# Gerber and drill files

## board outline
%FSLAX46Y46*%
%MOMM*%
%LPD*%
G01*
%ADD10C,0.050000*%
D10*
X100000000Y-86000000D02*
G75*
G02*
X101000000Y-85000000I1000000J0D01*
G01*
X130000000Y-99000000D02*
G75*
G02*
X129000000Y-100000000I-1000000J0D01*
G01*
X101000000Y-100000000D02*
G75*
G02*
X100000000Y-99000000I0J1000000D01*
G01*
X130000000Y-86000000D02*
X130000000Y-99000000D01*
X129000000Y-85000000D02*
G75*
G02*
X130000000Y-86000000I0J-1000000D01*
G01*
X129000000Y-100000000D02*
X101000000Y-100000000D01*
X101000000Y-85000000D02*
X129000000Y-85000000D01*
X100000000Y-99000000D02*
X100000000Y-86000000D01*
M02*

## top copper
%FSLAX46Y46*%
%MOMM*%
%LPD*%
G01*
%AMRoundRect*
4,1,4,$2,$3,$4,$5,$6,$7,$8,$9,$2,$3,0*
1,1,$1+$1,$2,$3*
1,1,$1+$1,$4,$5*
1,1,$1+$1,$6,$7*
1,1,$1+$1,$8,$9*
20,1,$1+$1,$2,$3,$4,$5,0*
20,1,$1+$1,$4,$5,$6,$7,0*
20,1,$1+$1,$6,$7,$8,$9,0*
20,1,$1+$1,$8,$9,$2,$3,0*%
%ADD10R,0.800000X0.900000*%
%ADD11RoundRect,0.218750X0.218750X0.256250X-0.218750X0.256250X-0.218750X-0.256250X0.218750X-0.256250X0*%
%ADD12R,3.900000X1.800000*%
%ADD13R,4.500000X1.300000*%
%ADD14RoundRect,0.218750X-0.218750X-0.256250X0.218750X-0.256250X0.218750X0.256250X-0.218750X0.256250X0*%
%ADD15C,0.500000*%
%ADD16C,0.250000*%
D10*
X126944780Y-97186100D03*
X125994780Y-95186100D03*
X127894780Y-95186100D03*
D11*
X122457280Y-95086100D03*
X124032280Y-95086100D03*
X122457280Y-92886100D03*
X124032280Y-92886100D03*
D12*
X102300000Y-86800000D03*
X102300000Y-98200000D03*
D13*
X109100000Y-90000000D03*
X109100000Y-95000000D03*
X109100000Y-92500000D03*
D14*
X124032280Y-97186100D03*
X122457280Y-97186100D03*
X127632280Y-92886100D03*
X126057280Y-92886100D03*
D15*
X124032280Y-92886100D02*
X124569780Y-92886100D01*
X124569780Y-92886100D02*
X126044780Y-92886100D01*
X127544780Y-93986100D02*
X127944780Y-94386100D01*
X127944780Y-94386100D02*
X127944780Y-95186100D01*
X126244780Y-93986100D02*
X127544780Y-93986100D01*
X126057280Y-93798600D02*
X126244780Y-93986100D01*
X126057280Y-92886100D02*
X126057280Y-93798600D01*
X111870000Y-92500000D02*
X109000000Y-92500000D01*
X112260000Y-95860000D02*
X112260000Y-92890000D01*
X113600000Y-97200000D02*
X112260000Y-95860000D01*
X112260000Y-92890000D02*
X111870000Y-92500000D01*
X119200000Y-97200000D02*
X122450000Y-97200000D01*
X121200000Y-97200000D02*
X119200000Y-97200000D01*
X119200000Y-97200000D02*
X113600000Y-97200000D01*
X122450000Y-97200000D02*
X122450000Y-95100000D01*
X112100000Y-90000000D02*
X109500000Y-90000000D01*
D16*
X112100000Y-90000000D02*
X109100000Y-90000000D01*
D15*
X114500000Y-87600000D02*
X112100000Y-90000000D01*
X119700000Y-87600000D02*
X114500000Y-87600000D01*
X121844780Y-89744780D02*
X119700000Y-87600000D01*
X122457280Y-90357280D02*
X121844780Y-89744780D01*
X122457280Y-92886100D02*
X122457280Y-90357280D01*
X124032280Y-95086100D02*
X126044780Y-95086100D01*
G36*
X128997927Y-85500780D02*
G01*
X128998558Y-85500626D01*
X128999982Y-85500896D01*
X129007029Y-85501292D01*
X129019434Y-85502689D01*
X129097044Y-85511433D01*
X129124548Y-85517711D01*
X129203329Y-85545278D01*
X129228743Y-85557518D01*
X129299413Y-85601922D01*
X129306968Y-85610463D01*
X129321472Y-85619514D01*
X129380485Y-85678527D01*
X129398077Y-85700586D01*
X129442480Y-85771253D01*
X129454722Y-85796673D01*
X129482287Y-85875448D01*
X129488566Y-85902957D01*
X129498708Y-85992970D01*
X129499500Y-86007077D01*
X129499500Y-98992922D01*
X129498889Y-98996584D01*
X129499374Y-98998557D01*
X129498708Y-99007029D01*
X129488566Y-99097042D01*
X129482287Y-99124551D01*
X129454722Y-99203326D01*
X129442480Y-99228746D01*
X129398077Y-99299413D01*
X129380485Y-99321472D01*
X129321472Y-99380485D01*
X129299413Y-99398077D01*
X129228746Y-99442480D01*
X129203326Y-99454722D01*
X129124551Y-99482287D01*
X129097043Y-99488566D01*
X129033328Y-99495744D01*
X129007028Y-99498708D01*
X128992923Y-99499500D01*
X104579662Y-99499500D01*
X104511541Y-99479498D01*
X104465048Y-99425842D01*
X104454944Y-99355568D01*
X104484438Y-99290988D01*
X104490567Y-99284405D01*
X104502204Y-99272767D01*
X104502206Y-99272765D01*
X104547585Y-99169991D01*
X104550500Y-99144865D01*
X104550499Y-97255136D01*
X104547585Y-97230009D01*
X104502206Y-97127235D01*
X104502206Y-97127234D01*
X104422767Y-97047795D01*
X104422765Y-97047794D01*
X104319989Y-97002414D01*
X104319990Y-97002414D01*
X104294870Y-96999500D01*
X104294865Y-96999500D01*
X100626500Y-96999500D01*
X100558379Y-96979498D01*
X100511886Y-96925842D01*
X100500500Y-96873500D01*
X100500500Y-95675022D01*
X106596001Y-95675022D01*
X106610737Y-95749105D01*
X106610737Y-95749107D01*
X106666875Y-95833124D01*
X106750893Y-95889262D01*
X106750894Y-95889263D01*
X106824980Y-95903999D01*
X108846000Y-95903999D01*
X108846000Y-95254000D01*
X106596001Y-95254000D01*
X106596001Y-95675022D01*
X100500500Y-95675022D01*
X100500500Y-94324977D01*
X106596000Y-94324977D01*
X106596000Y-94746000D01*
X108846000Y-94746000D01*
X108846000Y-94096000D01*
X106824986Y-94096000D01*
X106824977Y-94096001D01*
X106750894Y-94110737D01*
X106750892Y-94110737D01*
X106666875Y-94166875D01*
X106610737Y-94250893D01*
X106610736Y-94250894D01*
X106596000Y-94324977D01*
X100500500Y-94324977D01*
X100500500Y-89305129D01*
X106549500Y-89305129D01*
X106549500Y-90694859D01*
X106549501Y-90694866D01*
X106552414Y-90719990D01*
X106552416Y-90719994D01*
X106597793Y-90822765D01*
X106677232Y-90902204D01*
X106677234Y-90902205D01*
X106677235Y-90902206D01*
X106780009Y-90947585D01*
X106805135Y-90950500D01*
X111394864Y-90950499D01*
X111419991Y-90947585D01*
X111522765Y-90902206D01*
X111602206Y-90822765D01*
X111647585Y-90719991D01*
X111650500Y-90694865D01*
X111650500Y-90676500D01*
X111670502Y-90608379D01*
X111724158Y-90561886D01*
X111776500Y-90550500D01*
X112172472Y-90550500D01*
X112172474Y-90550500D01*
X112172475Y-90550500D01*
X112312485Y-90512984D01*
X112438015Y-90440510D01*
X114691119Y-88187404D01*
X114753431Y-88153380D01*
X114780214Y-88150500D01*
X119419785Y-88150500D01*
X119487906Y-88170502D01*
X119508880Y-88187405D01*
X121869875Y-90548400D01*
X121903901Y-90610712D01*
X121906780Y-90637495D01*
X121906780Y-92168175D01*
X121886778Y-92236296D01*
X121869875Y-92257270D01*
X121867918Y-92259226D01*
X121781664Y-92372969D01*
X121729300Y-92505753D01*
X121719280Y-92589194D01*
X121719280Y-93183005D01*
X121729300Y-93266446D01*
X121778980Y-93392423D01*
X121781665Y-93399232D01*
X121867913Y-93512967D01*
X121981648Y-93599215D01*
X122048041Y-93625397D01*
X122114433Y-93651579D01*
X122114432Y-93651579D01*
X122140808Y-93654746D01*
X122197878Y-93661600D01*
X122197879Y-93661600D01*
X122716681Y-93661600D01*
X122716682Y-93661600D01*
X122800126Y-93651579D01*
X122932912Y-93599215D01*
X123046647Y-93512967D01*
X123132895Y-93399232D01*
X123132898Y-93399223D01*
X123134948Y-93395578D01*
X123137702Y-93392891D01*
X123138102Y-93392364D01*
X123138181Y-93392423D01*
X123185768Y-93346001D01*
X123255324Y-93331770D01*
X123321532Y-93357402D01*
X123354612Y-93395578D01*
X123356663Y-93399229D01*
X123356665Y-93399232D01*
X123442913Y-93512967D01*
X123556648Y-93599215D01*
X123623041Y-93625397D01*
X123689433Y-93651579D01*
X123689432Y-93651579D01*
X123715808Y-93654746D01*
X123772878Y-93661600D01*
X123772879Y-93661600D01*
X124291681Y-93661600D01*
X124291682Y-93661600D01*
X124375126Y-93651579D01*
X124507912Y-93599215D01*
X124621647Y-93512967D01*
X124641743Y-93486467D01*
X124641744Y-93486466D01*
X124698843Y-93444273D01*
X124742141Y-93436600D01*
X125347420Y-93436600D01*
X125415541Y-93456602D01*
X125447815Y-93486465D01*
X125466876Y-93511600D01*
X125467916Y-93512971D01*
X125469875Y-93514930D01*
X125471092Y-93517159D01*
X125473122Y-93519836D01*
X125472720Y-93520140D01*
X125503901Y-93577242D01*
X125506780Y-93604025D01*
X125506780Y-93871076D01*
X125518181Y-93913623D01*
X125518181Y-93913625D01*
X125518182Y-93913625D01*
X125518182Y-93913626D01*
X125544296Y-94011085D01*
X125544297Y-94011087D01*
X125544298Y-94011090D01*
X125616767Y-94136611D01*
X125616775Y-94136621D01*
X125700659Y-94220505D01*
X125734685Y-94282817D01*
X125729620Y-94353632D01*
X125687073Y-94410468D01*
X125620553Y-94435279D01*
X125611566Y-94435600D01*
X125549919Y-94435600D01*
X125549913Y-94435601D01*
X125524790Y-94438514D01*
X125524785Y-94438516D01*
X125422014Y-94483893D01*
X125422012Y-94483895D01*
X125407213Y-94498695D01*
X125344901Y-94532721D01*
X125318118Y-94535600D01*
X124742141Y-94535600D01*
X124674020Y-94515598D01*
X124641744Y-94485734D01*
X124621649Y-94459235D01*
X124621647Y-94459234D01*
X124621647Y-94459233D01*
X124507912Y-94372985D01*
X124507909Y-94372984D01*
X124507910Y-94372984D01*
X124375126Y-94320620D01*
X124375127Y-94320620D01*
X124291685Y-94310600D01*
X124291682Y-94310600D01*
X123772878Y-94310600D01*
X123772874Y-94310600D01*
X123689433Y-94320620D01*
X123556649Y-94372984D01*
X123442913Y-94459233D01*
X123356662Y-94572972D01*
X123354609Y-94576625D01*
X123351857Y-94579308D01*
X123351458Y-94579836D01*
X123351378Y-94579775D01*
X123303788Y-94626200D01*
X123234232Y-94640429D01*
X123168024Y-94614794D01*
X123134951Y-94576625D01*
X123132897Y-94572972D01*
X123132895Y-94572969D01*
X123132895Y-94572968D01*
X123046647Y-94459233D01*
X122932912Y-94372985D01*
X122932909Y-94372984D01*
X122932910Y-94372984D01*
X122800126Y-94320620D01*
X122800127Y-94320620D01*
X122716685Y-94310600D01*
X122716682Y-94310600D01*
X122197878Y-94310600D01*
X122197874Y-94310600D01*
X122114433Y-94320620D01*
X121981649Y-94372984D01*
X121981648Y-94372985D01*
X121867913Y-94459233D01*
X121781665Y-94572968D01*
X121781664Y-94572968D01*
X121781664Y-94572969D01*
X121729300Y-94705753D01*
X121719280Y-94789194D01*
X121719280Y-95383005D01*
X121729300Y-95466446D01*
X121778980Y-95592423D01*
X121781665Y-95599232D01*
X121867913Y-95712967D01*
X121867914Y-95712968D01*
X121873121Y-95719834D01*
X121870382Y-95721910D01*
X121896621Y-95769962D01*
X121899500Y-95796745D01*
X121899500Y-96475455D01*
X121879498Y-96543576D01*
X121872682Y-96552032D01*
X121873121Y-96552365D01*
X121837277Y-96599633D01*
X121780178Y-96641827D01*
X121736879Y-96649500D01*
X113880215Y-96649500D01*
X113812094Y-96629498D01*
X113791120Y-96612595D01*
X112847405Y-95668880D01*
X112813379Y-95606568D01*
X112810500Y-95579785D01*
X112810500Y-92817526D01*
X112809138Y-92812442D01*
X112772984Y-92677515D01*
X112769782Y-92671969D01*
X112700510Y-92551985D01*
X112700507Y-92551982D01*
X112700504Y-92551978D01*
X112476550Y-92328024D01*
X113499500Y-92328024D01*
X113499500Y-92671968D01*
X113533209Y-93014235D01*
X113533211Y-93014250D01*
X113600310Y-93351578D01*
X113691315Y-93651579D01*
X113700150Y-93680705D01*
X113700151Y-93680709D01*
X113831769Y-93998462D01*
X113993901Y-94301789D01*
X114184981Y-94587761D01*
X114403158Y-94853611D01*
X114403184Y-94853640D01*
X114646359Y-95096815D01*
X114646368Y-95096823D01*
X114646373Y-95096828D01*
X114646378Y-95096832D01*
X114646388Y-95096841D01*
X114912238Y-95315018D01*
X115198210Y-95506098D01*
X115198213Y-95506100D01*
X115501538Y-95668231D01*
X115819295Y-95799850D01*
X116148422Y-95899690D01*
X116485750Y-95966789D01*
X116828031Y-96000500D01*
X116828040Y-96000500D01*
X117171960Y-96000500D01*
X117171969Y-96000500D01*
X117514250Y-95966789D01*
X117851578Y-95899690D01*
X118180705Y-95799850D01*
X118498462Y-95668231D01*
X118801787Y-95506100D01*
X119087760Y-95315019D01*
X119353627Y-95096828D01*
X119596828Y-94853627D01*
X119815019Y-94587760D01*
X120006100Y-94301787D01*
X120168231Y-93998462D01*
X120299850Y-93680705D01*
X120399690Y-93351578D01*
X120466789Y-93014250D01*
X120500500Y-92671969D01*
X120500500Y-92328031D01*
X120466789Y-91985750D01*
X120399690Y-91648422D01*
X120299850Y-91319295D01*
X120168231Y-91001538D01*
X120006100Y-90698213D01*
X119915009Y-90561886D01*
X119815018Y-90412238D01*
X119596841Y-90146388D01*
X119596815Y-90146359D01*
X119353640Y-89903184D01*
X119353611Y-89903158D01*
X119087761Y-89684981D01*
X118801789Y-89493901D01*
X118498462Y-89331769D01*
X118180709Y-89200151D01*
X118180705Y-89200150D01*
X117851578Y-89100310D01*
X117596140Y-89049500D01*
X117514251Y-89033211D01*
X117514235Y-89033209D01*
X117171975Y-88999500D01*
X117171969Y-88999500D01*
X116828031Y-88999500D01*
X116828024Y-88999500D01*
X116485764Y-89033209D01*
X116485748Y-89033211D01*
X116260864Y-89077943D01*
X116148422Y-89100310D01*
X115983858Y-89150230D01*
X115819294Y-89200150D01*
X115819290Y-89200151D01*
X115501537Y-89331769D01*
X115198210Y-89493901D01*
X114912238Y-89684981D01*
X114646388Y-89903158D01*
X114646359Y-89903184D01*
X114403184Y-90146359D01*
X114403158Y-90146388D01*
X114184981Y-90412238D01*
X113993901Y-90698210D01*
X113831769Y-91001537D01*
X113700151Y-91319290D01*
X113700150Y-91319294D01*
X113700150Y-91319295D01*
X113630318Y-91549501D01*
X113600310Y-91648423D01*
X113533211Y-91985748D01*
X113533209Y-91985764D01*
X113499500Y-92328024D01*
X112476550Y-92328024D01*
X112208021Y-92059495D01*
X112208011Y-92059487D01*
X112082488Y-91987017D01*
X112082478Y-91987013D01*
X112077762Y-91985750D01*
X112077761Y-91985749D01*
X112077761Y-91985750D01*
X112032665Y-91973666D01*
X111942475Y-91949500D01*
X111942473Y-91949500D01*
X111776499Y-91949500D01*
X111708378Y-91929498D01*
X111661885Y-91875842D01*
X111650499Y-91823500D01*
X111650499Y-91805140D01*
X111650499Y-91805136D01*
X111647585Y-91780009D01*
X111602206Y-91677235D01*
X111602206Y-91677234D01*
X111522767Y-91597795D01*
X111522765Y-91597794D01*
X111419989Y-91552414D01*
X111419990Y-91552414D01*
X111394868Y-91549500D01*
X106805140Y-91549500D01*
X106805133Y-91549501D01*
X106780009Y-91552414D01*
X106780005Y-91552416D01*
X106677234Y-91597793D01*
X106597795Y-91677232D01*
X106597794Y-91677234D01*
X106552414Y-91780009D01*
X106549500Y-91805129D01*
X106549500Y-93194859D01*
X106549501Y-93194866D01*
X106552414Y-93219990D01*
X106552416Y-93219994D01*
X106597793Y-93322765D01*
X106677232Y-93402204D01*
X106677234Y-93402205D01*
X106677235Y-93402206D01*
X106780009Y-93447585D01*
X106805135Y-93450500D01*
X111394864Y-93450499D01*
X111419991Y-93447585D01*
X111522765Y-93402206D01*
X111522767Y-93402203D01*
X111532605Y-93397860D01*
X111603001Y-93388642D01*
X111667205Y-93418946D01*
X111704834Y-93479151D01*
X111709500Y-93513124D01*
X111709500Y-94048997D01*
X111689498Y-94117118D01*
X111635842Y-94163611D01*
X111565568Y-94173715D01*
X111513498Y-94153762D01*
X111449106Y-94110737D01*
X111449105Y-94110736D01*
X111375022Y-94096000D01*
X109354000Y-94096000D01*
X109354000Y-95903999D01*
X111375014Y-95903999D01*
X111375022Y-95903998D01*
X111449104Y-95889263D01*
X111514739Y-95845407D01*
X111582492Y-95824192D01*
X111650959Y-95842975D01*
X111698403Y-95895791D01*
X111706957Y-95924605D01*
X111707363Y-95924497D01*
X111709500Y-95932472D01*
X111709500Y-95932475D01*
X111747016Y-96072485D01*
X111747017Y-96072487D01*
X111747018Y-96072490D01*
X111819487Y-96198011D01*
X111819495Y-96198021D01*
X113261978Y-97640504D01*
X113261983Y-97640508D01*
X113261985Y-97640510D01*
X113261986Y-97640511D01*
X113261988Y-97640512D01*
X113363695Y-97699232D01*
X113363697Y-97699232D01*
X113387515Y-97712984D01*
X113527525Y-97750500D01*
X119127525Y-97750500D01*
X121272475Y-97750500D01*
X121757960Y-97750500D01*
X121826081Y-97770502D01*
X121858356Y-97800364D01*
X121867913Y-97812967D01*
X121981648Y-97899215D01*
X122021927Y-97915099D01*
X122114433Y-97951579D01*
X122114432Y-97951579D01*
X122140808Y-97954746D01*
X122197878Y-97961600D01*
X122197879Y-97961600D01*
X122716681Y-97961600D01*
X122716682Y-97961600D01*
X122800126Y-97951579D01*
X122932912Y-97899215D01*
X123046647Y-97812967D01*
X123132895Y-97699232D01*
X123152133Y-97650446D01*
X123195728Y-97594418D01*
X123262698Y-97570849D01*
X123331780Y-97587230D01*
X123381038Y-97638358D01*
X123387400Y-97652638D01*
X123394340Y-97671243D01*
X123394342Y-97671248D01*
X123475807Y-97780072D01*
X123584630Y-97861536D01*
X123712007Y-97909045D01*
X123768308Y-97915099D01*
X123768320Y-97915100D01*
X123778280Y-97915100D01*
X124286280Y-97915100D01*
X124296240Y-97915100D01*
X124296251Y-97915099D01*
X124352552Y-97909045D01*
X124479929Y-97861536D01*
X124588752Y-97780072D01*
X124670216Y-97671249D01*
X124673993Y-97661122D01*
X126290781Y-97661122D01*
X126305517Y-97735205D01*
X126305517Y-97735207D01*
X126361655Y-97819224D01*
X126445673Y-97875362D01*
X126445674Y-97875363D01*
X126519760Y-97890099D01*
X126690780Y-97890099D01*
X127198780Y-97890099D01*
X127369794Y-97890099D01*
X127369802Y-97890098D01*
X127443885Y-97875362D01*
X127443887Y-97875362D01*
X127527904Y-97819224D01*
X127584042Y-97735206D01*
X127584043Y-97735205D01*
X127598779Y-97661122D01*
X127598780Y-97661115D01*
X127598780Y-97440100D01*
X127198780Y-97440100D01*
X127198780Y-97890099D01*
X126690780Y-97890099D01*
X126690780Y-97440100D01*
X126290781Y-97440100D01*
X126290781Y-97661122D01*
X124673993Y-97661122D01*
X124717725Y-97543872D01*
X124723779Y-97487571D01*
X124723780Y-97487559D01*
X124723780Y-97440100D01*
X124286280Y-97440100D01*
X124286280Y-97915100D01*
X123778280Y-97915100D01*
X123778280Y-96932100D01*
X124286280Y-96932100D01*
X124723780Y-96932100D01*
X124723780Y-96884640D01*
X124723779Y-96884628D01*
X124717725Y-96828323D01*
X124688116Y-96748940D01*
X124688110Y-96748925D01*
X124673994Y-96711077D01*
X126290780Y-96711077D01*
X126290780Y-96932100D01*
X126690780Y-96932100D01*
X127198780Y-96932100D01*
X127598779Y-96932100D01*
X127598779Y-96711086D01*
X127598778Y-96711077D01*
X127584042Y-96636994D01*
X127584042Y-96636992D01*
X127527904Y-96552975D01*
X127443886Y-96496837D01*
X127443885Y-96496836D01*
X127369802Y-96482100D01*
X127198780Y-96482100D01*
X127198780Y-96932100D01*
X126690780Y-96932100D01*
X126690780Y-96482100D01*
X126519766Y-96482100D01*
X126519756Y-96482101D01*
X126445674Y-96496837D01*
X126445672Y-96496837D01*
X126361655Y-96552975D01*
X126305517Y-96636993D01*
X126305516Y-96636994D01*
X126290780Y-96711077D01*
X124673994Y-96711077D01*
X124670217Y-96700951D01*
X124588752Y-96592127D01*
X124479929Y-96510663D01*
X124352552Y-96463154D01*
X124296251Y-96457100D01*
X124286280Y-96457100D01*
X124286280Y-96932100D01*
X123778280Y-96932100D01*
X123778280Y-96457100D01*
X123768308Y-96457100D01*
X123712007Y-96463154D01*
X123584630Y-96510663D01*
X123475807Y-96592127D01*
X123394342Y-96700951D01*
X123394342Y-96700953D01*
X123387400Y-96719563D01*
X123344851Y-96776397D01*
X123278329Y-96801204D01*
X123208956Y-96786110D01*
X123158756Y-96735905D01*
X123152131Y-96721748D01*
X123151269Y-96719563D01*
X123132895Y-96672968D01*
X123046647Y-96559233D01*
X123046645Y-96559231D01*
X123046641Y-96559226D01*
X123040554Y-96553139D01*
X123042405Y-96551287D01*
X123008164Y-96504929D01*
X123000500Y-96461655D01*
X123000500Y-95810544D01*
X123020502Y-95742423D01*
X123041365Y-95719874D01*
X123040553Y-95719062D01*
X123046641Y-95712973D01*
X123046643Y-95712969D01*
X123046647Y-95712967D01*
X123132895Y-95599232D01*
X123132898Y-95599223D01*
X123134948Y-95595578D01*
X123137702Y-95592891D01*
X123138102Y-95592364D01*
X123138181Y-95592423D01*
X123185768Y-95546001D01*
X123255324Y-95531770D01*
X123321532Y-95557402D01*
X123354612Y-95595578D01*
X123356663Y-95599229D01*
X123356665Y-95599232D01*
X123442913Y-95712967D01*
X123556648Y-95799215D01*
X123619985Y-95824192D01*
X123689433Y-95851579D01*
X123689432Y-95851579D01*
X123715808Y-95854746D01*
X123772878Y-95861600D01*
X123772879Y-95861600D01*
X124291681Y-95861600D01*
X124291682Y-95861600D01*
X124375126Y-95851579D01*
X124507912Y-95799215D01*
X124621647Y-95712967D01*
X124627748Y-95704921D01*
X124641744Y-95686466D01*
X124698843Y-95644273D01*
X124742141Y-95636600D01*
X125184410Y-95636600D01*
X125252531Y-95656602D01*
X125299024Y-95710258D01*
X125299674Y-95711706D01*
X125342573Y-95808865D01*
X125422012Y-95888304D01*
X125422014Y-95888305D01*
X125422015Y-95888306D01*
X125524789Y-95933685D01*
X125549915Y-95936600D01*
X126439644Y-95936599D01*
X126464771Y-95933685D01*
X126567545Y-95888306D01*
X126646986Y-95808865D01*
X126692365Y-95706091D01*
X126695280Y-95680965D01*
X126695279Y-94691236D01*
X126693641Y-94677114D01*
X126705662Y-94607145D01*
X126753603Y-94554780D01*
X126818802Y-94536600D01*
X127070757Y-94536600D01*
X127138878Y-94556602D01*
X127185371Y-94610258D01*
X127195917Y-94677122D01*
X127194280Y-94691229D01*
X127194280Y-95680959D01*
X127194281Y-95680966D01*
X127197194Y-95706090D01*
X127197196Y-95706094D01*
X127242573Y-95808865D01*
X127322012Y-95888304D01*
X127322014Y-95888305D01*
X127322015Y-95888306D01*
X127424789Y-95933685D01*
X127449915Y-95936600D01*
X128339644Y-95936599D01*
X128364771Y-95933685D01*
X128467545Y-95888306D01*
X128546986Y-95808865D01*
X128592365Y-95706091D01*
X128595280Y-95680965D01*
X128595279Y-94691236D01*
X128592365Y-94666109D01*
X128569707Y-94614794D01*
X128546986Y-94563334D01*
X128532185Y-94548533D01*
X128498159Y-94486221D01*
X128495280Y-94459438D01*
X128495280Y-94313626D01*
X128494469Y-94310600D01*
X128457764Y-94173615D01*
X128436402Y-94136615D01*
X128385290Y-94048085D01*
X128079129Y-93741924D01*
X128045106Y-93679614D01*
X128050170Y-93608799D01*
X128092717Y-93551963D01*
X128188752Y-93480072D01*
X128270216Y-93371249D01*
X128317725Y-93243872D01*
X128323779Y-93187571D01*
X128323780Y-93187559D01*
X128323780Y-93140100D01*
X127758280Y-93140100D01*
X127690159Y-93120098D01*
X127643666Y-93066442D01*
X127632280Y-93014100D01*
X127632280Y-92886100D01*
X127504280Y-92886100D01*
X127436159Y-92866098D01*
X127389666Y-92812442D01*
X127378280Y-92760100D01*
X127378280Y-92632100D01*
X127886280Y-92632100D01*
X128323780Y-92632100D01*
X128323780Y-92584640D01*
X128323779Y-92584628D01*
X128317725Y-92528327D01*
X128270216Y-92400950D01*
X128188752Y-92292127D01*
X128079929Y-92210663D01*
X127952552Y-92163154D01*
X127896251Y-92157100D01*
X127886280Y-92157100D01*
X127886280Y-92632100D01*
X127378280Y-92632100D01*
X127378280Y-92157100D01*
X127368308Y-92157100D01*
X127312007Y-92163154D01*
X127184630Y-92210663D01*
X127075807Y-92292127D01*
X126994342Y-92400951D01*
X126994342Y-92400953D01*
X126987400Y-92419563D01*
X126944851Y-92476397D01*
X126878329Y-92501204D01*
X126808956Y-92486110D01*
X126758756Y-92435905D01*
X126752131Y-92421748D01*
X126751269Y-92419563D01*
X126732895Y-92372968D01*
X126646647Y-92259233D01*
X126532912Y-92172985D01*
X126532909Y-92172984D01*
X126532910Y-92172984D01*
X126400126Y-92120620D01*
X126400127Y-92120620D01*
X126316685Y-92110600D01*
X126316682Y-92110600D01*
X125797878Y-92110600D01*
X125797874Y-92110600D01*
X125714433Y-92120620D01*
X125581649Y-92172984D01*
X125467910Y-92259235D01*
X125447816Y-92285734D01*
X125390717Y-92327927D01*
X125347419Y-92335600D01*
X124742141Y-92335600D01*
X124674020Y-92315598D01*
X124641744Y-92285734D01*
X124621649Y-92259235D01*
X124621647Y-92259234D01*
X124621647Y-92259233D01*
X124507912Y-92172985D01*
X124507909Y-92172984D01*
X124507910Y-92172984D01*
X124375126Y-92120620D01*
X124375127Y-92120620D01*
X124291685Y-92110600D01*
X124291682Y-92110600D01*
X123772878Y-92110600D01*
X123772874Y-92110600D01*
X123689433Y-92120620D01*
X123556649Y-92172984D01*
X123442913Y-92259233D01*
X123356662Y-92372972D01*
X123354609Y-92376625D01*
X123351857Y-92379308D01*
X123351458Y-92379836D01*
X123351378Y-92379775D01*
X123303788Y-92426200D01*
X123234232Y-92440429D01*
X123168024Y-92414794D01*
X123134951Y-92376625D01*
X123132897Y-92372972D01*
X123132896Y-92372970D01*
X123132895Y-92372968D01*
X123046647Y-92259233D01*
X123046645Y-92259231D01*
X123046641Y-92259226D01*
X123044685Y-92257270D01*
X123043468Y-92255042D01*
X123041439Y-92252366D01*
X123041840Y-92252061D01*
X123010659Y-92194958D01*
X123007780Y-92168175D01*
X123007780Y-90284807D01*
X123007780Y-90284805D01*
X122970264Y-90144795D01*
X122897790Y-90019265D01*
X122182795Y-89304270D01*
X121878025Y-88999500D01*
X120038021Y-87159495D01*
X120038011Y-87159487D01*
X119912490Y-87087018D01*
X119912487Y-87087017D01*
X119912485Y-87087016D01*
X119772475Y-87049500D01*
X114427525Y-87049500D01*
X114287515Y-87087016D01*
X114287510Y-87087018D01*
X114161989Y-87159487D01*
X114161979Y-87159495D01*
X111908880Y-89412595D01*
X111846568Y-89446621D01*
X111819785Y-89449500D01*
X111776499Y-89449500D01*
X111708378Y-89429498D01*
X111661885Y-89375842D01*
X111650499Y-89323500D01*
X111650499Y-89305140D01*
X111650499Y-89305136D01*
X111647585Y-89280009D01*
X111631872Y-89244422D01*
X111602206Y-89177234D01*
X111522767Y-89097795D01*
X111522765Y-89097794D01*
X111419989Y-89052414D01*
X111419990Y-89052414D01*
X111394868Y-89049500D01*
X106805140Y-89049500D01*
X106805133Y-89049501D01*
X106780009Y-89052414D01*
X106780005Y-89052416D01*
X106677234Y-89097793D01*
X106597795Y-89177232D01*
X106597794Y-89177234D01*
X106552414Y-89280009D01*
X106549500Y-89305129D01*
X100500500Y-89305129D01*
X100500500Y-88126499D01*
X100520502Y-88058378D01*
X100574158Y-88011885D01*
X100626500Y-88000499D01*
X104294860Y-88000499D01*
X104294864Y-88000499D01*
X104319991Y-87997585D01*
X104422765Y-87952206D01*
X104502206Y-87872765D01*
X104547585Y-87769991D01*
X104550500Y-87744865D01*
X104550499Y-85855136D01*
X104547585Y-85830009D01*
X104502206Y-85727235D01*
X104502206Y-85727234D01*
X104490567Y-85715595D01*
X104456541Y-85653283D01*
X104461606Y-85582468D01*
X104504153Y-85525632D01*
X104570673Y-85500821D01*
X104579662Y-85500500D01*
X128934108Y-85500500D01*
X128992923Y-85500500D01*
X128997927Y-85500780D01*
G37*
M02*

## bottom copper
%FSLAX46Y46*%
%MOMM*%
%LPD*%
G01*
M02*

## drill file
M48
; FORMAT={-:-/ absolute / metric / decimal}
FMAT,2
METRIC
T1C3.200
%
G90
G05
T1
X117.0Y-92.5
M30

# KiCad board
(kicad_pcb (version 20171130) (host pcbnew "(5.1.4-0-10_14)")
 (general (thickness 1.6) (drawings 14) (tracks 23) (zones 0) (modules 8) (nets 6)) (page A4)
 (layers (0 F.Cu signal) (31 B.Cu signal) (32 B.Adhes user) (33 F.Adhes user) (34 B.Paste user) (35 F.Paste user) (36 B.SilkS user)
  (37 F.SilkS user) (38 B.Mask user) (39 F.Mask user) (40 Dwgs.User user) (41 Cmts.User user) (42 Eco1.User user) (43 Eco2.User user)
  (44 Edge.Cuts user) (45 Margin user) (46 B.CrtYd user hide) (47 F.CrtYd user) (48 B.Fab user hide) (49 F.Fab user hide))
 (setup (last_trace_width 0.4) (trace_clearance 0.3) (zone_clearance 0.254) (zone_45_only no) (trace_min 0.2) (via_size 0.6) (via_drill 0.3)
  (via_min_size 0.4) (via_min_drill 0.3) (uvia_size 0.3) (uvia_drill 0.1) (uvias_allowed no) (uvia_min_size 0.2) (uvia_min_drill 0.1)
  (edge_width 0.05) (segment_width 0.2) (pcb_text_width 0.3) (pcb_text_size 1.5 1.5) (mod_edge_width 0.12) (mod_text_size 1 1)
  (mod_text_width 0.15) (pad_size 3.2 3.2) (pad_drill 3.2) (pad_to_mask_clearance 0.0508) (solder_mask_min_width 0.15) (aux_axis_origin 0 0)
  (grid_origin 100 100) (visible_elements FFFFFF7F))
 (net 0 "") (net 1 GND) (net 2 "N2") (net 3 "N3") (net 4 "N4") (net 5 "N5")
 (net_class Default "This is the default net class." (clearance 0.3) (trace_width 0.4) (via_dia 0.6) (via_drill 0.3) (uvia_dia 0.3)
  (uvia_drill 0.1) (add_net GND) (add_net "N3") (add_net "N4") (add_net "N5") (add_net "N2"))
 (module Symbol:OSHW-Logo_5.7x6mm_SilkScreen (layer F.Cu) (at 126.525 88.275)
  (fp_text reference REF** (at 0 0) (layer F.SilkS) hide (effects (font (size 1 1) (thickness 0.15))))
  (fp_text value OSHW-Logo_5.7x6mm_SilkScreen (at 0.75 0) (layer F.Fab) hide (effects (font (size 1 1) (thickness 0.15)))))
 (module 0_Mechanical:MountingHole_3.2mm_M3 (layer F.Cu) (at 117 92.5) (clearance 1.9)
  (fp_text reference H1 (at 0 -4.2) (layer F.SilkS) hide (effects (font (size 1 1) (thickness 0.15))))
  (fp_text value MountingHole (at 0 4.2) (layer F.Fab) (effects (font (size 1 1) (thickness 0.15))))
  (pad 1 np_thru_hole circle (at 0 0) (size 3.2 3.2) (drill 3.2) (layers *.Cu *.Mask)))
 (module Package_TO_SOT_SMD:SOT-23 (layer F.Cu) (at 126.94478 96.1861 270)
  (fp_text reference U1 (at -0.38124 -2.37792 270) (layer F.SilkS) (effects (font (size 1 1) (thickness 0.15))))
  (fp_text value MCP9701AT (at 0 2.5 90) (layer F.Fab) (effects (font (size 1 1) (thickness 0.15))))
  (pad 3 smd rect (at 1 0 270) (size 0.9 0.8) (layers F.Cu F.Paste F.Mask) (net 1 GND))
  (pad 2 smd rect (at -1 0.95 270) (size 0.9 0.8) (layers F.Cu F.Paste F.Mask) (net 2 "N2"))
  (pad 1 smd rect (at -1 -0.95 270) (size 0.9 0.8) (layers F.Cu F.Paste F.Mask) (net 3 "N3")))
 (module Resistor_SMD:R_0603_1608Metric (layer F.Cu) (at 123.24478 95.0861 180)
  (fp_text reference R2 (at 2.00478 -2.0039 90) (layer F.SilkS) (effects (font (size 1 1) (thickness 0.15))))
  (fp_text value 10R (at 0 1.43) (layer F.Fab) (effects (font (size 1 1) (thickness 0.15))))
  (pad 2 smd roundrect (at 0.7875 0 180) (size 0.875 0.95) (layers F.Cu F.Paste F.Mask) (roundrect_rratio 0.25) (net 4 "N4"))
  (pad 1 smd roundrect (at -0.7875 0 180) (size 0.875 0.95) (layers F.Cu F.Paste F.Mask) (roundrect_rratio 0.25) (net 2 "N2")))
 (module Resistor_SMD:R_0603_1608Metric (layer F.Cu) (at 123.24478 92.8861 180)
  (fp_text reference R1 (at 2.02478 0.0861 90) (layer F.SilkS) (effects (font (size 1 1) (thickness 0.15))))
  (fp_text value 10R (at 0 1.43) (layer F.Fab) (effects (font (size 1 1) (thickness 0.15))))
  (pad 2 smd roundrect (at 0.7875 0 180) (size 0.875 0.95) (layers F.Cu F.Paste F.Mask) (roundrect_rratio 0.25) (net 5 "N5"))
  (pad 1 smd roundrect (at -0.7875 0 180) (size 0.875 0.95) (layers F.Cu F.Paste F.Mask) (roundrect_rratio 0.25) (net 3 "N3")))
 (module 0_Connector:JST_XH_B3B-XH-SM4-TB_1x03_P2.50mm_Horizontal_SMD (layer F.Cu) (at 109.1 92.5 270)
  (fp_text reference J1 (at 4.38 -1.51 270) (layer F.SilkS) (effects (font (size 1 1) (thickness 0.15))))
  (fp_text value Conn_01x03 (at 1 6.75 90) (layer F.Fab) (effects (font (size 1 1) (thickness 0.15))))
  (pad "" smd rect (at -5.7 6.8 270) (size 1.8 3.9) (layers F.Cu F.Paste F.Mask))
  (pad "" smd rect (at 5.7 6.8 270) (size 1.8 3.9) (layers F.Cu F.Paste F.Mask))
  (pad 1 smd rect (at -2.5 0 270) (size 1.3 4.5) (layers F.Cu F.Paste F.Mask) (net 5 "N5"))
  (pad 3 smd rect (at 2.5 0 270) (size 1.3 4.5) (layers F.Cu F.Paste F.Mask) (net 1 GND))
  (pad 2 smd rect (at 0 0 270) (size 1.3 4.5) (layers F.Cu F.Paste F.Mask) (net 4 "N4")))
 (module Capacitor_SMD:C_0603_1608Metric (layer F.Cu) (at 123.24478 97.1861)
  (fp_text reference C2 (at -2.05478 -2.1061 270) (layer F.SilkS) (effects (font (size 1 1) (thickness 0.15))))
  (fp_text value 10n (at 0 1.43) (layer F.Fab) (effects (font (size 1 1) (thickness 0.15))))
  (pad 2 smd roundrect (at 0.7875 0) (size 0.875 0.95) (layers F.Cu F.Paste F.Mask) (roundrect_rratio 0.25) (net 1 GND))
  (pad 1 smd roundrect (at -0.7875 0) (size 0.875 0.95) (layers F.Cu F.Paste F.Mask) (roundrect_rratio 0.25) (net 4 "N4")))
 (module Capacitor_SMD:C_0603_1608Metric (layer F.Cu) (at 126.84478 92.8861)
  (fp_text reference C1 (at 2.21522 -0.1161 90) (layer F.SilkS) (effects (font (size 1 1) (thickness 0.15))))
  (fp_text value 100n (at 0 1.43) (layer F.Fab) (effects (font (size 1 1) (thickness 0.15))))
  (pad 2 smd roundrect (at 0.7875 0) (size 0.875 0.95) (layers F.Cu F.Paste F.Mask) (roundrect_rratio 0.25) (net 1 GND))
  (pad 1 smd roundrect (at -0.7875 0) (size 0.875 0.95) (layers F.Cu F.Paste F.Mask) (roundrect_rratio 0.25) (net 3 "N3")))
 (gr_arc (start 101 86) (end 101 85) (angle -90) (layer Edge.Cuts) (width 0.05))
 (gr_arc (start 129 99) (end 129 100) (angle -90) (layer Edge.Cuts) (width 0.05))
 (gr_arc (start 101 99) (end 100 99) (angle -90) (layer Edge.Cuts) (width 0.05))
 (gr_line (start 130 86) (end 130 99) (layer Edge.Cuts) (width 0.05))
 (gr_arc (start 129 86) (end 130 86) (angle -90) (layer Edge.Cuts) (width 0.05))
 (gr_line (start 129 100) (end 101 100) (layer Edge.Cuts) (width 0.05))
 (gr_line (start 101 85) (end 129 85) (layer Edge.Cuts) (width 0.05))
 (gr_line (start 100 99) (end 100 86) (layer Edge.Cuts) (width 0.05))
 (segment (start 124.03228 92.8861) (end 124.56978 92.8861) (width 0.5) (layer F.Cu) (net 3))
 (segment (start 124.56978 92.8861) (end 126.04478 92.8861) (width 0.5) (layer F.Cu) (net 3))
 (segment (start 127.54478 93.9861) (end 127.94478 94.3861) (width 0.5) (layer F.Cu) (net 3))
 (segment (start 127.94478 94.3861) (end 127.94478 95.1861) (width 0.5) (layer F.Cu) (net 3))
 (segment (start 126.24478 93.9861) (end 127.54478 93.9861) (width 0.5) (layer F.Cu) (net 3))
 (segment (start 126.05728 93.7986) (end 126.24478 93.9861) (width 0.5) (layer F.Cu) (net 3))
 (segment (start 126.05728 92.8861) (end 126.05728 93.7986) (width 0.5) (layer F.Cu) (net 3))
 (segment (start 111.87 92.5) (end 109 92.5) (width 0.5) (layer F.Cu) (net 4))
 (segment (start 112.26 95.86) (end 112.26 92.89) (width 0.5) (layer F.Cu) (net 4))
 (segment (start 113.6 97.2) (end 112.26 95.86) (width 0.5) (layer F.Cu) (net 4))
 (segment (start 112.26 92.89) (end 111.87 92.5) (width 0.5) (layer F.Cu) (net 4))
 (segment (start 119.2 97.2) (end 122.45 97.2) (width 0.5) (layer F.Cu) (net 4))
 (segment (start 121.2 97.2) (end 119.2 97.2) (width 0.5) (layer F.Cu) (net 4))
 (segment (start 119.2 97.2) (end 113.6 97.2) (width 0.5) (layer F.Cu) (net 4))
 (segment (start 122.45 97.2) (end 122.45 95.1) (width 0.5) (layer F.Cu) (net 4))
 (segment (start 112.1 90) (end 109.5 90) (width 0.5) (layer F.Cu) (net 5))
 (segment (start 112.1 90) (end 109.1 90) (width 0.25) (layer F.Cu) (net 5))
 (segment (start 114.5 87.6) (end 112.1 90) (width 0.5) (layer F.Cu) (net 5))
 (segment (start 119.7 87.6) (end 114.5 87.6) (width 0.5) (layer F.Cu) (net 5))
 (segment (start 121.84478 89.74478) (end 119.7 87.6) (width 0.5) (layer F.Cu) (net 5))
 (segment (start 122.45728 90.35728) (end 121.84478 89.74478) (width 0.5) (layer F.Cu) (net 5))
 (segment (start 122.45728 92.8861) (end 122.45728 90.35728) (width 0.5) (layer F.Cu) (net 5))
 (segment (start 124.03228 95.0861) (end 126.04478 95.0861) (width 0.5) (layer F.Cu) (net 2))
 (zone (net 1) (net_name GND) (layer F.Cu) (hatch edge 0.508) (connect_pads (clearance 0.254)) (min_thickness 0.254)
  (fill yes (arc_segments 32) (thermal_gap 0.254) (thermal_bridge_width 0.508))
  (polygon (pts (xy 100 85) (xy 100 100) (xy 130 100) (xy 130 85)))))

